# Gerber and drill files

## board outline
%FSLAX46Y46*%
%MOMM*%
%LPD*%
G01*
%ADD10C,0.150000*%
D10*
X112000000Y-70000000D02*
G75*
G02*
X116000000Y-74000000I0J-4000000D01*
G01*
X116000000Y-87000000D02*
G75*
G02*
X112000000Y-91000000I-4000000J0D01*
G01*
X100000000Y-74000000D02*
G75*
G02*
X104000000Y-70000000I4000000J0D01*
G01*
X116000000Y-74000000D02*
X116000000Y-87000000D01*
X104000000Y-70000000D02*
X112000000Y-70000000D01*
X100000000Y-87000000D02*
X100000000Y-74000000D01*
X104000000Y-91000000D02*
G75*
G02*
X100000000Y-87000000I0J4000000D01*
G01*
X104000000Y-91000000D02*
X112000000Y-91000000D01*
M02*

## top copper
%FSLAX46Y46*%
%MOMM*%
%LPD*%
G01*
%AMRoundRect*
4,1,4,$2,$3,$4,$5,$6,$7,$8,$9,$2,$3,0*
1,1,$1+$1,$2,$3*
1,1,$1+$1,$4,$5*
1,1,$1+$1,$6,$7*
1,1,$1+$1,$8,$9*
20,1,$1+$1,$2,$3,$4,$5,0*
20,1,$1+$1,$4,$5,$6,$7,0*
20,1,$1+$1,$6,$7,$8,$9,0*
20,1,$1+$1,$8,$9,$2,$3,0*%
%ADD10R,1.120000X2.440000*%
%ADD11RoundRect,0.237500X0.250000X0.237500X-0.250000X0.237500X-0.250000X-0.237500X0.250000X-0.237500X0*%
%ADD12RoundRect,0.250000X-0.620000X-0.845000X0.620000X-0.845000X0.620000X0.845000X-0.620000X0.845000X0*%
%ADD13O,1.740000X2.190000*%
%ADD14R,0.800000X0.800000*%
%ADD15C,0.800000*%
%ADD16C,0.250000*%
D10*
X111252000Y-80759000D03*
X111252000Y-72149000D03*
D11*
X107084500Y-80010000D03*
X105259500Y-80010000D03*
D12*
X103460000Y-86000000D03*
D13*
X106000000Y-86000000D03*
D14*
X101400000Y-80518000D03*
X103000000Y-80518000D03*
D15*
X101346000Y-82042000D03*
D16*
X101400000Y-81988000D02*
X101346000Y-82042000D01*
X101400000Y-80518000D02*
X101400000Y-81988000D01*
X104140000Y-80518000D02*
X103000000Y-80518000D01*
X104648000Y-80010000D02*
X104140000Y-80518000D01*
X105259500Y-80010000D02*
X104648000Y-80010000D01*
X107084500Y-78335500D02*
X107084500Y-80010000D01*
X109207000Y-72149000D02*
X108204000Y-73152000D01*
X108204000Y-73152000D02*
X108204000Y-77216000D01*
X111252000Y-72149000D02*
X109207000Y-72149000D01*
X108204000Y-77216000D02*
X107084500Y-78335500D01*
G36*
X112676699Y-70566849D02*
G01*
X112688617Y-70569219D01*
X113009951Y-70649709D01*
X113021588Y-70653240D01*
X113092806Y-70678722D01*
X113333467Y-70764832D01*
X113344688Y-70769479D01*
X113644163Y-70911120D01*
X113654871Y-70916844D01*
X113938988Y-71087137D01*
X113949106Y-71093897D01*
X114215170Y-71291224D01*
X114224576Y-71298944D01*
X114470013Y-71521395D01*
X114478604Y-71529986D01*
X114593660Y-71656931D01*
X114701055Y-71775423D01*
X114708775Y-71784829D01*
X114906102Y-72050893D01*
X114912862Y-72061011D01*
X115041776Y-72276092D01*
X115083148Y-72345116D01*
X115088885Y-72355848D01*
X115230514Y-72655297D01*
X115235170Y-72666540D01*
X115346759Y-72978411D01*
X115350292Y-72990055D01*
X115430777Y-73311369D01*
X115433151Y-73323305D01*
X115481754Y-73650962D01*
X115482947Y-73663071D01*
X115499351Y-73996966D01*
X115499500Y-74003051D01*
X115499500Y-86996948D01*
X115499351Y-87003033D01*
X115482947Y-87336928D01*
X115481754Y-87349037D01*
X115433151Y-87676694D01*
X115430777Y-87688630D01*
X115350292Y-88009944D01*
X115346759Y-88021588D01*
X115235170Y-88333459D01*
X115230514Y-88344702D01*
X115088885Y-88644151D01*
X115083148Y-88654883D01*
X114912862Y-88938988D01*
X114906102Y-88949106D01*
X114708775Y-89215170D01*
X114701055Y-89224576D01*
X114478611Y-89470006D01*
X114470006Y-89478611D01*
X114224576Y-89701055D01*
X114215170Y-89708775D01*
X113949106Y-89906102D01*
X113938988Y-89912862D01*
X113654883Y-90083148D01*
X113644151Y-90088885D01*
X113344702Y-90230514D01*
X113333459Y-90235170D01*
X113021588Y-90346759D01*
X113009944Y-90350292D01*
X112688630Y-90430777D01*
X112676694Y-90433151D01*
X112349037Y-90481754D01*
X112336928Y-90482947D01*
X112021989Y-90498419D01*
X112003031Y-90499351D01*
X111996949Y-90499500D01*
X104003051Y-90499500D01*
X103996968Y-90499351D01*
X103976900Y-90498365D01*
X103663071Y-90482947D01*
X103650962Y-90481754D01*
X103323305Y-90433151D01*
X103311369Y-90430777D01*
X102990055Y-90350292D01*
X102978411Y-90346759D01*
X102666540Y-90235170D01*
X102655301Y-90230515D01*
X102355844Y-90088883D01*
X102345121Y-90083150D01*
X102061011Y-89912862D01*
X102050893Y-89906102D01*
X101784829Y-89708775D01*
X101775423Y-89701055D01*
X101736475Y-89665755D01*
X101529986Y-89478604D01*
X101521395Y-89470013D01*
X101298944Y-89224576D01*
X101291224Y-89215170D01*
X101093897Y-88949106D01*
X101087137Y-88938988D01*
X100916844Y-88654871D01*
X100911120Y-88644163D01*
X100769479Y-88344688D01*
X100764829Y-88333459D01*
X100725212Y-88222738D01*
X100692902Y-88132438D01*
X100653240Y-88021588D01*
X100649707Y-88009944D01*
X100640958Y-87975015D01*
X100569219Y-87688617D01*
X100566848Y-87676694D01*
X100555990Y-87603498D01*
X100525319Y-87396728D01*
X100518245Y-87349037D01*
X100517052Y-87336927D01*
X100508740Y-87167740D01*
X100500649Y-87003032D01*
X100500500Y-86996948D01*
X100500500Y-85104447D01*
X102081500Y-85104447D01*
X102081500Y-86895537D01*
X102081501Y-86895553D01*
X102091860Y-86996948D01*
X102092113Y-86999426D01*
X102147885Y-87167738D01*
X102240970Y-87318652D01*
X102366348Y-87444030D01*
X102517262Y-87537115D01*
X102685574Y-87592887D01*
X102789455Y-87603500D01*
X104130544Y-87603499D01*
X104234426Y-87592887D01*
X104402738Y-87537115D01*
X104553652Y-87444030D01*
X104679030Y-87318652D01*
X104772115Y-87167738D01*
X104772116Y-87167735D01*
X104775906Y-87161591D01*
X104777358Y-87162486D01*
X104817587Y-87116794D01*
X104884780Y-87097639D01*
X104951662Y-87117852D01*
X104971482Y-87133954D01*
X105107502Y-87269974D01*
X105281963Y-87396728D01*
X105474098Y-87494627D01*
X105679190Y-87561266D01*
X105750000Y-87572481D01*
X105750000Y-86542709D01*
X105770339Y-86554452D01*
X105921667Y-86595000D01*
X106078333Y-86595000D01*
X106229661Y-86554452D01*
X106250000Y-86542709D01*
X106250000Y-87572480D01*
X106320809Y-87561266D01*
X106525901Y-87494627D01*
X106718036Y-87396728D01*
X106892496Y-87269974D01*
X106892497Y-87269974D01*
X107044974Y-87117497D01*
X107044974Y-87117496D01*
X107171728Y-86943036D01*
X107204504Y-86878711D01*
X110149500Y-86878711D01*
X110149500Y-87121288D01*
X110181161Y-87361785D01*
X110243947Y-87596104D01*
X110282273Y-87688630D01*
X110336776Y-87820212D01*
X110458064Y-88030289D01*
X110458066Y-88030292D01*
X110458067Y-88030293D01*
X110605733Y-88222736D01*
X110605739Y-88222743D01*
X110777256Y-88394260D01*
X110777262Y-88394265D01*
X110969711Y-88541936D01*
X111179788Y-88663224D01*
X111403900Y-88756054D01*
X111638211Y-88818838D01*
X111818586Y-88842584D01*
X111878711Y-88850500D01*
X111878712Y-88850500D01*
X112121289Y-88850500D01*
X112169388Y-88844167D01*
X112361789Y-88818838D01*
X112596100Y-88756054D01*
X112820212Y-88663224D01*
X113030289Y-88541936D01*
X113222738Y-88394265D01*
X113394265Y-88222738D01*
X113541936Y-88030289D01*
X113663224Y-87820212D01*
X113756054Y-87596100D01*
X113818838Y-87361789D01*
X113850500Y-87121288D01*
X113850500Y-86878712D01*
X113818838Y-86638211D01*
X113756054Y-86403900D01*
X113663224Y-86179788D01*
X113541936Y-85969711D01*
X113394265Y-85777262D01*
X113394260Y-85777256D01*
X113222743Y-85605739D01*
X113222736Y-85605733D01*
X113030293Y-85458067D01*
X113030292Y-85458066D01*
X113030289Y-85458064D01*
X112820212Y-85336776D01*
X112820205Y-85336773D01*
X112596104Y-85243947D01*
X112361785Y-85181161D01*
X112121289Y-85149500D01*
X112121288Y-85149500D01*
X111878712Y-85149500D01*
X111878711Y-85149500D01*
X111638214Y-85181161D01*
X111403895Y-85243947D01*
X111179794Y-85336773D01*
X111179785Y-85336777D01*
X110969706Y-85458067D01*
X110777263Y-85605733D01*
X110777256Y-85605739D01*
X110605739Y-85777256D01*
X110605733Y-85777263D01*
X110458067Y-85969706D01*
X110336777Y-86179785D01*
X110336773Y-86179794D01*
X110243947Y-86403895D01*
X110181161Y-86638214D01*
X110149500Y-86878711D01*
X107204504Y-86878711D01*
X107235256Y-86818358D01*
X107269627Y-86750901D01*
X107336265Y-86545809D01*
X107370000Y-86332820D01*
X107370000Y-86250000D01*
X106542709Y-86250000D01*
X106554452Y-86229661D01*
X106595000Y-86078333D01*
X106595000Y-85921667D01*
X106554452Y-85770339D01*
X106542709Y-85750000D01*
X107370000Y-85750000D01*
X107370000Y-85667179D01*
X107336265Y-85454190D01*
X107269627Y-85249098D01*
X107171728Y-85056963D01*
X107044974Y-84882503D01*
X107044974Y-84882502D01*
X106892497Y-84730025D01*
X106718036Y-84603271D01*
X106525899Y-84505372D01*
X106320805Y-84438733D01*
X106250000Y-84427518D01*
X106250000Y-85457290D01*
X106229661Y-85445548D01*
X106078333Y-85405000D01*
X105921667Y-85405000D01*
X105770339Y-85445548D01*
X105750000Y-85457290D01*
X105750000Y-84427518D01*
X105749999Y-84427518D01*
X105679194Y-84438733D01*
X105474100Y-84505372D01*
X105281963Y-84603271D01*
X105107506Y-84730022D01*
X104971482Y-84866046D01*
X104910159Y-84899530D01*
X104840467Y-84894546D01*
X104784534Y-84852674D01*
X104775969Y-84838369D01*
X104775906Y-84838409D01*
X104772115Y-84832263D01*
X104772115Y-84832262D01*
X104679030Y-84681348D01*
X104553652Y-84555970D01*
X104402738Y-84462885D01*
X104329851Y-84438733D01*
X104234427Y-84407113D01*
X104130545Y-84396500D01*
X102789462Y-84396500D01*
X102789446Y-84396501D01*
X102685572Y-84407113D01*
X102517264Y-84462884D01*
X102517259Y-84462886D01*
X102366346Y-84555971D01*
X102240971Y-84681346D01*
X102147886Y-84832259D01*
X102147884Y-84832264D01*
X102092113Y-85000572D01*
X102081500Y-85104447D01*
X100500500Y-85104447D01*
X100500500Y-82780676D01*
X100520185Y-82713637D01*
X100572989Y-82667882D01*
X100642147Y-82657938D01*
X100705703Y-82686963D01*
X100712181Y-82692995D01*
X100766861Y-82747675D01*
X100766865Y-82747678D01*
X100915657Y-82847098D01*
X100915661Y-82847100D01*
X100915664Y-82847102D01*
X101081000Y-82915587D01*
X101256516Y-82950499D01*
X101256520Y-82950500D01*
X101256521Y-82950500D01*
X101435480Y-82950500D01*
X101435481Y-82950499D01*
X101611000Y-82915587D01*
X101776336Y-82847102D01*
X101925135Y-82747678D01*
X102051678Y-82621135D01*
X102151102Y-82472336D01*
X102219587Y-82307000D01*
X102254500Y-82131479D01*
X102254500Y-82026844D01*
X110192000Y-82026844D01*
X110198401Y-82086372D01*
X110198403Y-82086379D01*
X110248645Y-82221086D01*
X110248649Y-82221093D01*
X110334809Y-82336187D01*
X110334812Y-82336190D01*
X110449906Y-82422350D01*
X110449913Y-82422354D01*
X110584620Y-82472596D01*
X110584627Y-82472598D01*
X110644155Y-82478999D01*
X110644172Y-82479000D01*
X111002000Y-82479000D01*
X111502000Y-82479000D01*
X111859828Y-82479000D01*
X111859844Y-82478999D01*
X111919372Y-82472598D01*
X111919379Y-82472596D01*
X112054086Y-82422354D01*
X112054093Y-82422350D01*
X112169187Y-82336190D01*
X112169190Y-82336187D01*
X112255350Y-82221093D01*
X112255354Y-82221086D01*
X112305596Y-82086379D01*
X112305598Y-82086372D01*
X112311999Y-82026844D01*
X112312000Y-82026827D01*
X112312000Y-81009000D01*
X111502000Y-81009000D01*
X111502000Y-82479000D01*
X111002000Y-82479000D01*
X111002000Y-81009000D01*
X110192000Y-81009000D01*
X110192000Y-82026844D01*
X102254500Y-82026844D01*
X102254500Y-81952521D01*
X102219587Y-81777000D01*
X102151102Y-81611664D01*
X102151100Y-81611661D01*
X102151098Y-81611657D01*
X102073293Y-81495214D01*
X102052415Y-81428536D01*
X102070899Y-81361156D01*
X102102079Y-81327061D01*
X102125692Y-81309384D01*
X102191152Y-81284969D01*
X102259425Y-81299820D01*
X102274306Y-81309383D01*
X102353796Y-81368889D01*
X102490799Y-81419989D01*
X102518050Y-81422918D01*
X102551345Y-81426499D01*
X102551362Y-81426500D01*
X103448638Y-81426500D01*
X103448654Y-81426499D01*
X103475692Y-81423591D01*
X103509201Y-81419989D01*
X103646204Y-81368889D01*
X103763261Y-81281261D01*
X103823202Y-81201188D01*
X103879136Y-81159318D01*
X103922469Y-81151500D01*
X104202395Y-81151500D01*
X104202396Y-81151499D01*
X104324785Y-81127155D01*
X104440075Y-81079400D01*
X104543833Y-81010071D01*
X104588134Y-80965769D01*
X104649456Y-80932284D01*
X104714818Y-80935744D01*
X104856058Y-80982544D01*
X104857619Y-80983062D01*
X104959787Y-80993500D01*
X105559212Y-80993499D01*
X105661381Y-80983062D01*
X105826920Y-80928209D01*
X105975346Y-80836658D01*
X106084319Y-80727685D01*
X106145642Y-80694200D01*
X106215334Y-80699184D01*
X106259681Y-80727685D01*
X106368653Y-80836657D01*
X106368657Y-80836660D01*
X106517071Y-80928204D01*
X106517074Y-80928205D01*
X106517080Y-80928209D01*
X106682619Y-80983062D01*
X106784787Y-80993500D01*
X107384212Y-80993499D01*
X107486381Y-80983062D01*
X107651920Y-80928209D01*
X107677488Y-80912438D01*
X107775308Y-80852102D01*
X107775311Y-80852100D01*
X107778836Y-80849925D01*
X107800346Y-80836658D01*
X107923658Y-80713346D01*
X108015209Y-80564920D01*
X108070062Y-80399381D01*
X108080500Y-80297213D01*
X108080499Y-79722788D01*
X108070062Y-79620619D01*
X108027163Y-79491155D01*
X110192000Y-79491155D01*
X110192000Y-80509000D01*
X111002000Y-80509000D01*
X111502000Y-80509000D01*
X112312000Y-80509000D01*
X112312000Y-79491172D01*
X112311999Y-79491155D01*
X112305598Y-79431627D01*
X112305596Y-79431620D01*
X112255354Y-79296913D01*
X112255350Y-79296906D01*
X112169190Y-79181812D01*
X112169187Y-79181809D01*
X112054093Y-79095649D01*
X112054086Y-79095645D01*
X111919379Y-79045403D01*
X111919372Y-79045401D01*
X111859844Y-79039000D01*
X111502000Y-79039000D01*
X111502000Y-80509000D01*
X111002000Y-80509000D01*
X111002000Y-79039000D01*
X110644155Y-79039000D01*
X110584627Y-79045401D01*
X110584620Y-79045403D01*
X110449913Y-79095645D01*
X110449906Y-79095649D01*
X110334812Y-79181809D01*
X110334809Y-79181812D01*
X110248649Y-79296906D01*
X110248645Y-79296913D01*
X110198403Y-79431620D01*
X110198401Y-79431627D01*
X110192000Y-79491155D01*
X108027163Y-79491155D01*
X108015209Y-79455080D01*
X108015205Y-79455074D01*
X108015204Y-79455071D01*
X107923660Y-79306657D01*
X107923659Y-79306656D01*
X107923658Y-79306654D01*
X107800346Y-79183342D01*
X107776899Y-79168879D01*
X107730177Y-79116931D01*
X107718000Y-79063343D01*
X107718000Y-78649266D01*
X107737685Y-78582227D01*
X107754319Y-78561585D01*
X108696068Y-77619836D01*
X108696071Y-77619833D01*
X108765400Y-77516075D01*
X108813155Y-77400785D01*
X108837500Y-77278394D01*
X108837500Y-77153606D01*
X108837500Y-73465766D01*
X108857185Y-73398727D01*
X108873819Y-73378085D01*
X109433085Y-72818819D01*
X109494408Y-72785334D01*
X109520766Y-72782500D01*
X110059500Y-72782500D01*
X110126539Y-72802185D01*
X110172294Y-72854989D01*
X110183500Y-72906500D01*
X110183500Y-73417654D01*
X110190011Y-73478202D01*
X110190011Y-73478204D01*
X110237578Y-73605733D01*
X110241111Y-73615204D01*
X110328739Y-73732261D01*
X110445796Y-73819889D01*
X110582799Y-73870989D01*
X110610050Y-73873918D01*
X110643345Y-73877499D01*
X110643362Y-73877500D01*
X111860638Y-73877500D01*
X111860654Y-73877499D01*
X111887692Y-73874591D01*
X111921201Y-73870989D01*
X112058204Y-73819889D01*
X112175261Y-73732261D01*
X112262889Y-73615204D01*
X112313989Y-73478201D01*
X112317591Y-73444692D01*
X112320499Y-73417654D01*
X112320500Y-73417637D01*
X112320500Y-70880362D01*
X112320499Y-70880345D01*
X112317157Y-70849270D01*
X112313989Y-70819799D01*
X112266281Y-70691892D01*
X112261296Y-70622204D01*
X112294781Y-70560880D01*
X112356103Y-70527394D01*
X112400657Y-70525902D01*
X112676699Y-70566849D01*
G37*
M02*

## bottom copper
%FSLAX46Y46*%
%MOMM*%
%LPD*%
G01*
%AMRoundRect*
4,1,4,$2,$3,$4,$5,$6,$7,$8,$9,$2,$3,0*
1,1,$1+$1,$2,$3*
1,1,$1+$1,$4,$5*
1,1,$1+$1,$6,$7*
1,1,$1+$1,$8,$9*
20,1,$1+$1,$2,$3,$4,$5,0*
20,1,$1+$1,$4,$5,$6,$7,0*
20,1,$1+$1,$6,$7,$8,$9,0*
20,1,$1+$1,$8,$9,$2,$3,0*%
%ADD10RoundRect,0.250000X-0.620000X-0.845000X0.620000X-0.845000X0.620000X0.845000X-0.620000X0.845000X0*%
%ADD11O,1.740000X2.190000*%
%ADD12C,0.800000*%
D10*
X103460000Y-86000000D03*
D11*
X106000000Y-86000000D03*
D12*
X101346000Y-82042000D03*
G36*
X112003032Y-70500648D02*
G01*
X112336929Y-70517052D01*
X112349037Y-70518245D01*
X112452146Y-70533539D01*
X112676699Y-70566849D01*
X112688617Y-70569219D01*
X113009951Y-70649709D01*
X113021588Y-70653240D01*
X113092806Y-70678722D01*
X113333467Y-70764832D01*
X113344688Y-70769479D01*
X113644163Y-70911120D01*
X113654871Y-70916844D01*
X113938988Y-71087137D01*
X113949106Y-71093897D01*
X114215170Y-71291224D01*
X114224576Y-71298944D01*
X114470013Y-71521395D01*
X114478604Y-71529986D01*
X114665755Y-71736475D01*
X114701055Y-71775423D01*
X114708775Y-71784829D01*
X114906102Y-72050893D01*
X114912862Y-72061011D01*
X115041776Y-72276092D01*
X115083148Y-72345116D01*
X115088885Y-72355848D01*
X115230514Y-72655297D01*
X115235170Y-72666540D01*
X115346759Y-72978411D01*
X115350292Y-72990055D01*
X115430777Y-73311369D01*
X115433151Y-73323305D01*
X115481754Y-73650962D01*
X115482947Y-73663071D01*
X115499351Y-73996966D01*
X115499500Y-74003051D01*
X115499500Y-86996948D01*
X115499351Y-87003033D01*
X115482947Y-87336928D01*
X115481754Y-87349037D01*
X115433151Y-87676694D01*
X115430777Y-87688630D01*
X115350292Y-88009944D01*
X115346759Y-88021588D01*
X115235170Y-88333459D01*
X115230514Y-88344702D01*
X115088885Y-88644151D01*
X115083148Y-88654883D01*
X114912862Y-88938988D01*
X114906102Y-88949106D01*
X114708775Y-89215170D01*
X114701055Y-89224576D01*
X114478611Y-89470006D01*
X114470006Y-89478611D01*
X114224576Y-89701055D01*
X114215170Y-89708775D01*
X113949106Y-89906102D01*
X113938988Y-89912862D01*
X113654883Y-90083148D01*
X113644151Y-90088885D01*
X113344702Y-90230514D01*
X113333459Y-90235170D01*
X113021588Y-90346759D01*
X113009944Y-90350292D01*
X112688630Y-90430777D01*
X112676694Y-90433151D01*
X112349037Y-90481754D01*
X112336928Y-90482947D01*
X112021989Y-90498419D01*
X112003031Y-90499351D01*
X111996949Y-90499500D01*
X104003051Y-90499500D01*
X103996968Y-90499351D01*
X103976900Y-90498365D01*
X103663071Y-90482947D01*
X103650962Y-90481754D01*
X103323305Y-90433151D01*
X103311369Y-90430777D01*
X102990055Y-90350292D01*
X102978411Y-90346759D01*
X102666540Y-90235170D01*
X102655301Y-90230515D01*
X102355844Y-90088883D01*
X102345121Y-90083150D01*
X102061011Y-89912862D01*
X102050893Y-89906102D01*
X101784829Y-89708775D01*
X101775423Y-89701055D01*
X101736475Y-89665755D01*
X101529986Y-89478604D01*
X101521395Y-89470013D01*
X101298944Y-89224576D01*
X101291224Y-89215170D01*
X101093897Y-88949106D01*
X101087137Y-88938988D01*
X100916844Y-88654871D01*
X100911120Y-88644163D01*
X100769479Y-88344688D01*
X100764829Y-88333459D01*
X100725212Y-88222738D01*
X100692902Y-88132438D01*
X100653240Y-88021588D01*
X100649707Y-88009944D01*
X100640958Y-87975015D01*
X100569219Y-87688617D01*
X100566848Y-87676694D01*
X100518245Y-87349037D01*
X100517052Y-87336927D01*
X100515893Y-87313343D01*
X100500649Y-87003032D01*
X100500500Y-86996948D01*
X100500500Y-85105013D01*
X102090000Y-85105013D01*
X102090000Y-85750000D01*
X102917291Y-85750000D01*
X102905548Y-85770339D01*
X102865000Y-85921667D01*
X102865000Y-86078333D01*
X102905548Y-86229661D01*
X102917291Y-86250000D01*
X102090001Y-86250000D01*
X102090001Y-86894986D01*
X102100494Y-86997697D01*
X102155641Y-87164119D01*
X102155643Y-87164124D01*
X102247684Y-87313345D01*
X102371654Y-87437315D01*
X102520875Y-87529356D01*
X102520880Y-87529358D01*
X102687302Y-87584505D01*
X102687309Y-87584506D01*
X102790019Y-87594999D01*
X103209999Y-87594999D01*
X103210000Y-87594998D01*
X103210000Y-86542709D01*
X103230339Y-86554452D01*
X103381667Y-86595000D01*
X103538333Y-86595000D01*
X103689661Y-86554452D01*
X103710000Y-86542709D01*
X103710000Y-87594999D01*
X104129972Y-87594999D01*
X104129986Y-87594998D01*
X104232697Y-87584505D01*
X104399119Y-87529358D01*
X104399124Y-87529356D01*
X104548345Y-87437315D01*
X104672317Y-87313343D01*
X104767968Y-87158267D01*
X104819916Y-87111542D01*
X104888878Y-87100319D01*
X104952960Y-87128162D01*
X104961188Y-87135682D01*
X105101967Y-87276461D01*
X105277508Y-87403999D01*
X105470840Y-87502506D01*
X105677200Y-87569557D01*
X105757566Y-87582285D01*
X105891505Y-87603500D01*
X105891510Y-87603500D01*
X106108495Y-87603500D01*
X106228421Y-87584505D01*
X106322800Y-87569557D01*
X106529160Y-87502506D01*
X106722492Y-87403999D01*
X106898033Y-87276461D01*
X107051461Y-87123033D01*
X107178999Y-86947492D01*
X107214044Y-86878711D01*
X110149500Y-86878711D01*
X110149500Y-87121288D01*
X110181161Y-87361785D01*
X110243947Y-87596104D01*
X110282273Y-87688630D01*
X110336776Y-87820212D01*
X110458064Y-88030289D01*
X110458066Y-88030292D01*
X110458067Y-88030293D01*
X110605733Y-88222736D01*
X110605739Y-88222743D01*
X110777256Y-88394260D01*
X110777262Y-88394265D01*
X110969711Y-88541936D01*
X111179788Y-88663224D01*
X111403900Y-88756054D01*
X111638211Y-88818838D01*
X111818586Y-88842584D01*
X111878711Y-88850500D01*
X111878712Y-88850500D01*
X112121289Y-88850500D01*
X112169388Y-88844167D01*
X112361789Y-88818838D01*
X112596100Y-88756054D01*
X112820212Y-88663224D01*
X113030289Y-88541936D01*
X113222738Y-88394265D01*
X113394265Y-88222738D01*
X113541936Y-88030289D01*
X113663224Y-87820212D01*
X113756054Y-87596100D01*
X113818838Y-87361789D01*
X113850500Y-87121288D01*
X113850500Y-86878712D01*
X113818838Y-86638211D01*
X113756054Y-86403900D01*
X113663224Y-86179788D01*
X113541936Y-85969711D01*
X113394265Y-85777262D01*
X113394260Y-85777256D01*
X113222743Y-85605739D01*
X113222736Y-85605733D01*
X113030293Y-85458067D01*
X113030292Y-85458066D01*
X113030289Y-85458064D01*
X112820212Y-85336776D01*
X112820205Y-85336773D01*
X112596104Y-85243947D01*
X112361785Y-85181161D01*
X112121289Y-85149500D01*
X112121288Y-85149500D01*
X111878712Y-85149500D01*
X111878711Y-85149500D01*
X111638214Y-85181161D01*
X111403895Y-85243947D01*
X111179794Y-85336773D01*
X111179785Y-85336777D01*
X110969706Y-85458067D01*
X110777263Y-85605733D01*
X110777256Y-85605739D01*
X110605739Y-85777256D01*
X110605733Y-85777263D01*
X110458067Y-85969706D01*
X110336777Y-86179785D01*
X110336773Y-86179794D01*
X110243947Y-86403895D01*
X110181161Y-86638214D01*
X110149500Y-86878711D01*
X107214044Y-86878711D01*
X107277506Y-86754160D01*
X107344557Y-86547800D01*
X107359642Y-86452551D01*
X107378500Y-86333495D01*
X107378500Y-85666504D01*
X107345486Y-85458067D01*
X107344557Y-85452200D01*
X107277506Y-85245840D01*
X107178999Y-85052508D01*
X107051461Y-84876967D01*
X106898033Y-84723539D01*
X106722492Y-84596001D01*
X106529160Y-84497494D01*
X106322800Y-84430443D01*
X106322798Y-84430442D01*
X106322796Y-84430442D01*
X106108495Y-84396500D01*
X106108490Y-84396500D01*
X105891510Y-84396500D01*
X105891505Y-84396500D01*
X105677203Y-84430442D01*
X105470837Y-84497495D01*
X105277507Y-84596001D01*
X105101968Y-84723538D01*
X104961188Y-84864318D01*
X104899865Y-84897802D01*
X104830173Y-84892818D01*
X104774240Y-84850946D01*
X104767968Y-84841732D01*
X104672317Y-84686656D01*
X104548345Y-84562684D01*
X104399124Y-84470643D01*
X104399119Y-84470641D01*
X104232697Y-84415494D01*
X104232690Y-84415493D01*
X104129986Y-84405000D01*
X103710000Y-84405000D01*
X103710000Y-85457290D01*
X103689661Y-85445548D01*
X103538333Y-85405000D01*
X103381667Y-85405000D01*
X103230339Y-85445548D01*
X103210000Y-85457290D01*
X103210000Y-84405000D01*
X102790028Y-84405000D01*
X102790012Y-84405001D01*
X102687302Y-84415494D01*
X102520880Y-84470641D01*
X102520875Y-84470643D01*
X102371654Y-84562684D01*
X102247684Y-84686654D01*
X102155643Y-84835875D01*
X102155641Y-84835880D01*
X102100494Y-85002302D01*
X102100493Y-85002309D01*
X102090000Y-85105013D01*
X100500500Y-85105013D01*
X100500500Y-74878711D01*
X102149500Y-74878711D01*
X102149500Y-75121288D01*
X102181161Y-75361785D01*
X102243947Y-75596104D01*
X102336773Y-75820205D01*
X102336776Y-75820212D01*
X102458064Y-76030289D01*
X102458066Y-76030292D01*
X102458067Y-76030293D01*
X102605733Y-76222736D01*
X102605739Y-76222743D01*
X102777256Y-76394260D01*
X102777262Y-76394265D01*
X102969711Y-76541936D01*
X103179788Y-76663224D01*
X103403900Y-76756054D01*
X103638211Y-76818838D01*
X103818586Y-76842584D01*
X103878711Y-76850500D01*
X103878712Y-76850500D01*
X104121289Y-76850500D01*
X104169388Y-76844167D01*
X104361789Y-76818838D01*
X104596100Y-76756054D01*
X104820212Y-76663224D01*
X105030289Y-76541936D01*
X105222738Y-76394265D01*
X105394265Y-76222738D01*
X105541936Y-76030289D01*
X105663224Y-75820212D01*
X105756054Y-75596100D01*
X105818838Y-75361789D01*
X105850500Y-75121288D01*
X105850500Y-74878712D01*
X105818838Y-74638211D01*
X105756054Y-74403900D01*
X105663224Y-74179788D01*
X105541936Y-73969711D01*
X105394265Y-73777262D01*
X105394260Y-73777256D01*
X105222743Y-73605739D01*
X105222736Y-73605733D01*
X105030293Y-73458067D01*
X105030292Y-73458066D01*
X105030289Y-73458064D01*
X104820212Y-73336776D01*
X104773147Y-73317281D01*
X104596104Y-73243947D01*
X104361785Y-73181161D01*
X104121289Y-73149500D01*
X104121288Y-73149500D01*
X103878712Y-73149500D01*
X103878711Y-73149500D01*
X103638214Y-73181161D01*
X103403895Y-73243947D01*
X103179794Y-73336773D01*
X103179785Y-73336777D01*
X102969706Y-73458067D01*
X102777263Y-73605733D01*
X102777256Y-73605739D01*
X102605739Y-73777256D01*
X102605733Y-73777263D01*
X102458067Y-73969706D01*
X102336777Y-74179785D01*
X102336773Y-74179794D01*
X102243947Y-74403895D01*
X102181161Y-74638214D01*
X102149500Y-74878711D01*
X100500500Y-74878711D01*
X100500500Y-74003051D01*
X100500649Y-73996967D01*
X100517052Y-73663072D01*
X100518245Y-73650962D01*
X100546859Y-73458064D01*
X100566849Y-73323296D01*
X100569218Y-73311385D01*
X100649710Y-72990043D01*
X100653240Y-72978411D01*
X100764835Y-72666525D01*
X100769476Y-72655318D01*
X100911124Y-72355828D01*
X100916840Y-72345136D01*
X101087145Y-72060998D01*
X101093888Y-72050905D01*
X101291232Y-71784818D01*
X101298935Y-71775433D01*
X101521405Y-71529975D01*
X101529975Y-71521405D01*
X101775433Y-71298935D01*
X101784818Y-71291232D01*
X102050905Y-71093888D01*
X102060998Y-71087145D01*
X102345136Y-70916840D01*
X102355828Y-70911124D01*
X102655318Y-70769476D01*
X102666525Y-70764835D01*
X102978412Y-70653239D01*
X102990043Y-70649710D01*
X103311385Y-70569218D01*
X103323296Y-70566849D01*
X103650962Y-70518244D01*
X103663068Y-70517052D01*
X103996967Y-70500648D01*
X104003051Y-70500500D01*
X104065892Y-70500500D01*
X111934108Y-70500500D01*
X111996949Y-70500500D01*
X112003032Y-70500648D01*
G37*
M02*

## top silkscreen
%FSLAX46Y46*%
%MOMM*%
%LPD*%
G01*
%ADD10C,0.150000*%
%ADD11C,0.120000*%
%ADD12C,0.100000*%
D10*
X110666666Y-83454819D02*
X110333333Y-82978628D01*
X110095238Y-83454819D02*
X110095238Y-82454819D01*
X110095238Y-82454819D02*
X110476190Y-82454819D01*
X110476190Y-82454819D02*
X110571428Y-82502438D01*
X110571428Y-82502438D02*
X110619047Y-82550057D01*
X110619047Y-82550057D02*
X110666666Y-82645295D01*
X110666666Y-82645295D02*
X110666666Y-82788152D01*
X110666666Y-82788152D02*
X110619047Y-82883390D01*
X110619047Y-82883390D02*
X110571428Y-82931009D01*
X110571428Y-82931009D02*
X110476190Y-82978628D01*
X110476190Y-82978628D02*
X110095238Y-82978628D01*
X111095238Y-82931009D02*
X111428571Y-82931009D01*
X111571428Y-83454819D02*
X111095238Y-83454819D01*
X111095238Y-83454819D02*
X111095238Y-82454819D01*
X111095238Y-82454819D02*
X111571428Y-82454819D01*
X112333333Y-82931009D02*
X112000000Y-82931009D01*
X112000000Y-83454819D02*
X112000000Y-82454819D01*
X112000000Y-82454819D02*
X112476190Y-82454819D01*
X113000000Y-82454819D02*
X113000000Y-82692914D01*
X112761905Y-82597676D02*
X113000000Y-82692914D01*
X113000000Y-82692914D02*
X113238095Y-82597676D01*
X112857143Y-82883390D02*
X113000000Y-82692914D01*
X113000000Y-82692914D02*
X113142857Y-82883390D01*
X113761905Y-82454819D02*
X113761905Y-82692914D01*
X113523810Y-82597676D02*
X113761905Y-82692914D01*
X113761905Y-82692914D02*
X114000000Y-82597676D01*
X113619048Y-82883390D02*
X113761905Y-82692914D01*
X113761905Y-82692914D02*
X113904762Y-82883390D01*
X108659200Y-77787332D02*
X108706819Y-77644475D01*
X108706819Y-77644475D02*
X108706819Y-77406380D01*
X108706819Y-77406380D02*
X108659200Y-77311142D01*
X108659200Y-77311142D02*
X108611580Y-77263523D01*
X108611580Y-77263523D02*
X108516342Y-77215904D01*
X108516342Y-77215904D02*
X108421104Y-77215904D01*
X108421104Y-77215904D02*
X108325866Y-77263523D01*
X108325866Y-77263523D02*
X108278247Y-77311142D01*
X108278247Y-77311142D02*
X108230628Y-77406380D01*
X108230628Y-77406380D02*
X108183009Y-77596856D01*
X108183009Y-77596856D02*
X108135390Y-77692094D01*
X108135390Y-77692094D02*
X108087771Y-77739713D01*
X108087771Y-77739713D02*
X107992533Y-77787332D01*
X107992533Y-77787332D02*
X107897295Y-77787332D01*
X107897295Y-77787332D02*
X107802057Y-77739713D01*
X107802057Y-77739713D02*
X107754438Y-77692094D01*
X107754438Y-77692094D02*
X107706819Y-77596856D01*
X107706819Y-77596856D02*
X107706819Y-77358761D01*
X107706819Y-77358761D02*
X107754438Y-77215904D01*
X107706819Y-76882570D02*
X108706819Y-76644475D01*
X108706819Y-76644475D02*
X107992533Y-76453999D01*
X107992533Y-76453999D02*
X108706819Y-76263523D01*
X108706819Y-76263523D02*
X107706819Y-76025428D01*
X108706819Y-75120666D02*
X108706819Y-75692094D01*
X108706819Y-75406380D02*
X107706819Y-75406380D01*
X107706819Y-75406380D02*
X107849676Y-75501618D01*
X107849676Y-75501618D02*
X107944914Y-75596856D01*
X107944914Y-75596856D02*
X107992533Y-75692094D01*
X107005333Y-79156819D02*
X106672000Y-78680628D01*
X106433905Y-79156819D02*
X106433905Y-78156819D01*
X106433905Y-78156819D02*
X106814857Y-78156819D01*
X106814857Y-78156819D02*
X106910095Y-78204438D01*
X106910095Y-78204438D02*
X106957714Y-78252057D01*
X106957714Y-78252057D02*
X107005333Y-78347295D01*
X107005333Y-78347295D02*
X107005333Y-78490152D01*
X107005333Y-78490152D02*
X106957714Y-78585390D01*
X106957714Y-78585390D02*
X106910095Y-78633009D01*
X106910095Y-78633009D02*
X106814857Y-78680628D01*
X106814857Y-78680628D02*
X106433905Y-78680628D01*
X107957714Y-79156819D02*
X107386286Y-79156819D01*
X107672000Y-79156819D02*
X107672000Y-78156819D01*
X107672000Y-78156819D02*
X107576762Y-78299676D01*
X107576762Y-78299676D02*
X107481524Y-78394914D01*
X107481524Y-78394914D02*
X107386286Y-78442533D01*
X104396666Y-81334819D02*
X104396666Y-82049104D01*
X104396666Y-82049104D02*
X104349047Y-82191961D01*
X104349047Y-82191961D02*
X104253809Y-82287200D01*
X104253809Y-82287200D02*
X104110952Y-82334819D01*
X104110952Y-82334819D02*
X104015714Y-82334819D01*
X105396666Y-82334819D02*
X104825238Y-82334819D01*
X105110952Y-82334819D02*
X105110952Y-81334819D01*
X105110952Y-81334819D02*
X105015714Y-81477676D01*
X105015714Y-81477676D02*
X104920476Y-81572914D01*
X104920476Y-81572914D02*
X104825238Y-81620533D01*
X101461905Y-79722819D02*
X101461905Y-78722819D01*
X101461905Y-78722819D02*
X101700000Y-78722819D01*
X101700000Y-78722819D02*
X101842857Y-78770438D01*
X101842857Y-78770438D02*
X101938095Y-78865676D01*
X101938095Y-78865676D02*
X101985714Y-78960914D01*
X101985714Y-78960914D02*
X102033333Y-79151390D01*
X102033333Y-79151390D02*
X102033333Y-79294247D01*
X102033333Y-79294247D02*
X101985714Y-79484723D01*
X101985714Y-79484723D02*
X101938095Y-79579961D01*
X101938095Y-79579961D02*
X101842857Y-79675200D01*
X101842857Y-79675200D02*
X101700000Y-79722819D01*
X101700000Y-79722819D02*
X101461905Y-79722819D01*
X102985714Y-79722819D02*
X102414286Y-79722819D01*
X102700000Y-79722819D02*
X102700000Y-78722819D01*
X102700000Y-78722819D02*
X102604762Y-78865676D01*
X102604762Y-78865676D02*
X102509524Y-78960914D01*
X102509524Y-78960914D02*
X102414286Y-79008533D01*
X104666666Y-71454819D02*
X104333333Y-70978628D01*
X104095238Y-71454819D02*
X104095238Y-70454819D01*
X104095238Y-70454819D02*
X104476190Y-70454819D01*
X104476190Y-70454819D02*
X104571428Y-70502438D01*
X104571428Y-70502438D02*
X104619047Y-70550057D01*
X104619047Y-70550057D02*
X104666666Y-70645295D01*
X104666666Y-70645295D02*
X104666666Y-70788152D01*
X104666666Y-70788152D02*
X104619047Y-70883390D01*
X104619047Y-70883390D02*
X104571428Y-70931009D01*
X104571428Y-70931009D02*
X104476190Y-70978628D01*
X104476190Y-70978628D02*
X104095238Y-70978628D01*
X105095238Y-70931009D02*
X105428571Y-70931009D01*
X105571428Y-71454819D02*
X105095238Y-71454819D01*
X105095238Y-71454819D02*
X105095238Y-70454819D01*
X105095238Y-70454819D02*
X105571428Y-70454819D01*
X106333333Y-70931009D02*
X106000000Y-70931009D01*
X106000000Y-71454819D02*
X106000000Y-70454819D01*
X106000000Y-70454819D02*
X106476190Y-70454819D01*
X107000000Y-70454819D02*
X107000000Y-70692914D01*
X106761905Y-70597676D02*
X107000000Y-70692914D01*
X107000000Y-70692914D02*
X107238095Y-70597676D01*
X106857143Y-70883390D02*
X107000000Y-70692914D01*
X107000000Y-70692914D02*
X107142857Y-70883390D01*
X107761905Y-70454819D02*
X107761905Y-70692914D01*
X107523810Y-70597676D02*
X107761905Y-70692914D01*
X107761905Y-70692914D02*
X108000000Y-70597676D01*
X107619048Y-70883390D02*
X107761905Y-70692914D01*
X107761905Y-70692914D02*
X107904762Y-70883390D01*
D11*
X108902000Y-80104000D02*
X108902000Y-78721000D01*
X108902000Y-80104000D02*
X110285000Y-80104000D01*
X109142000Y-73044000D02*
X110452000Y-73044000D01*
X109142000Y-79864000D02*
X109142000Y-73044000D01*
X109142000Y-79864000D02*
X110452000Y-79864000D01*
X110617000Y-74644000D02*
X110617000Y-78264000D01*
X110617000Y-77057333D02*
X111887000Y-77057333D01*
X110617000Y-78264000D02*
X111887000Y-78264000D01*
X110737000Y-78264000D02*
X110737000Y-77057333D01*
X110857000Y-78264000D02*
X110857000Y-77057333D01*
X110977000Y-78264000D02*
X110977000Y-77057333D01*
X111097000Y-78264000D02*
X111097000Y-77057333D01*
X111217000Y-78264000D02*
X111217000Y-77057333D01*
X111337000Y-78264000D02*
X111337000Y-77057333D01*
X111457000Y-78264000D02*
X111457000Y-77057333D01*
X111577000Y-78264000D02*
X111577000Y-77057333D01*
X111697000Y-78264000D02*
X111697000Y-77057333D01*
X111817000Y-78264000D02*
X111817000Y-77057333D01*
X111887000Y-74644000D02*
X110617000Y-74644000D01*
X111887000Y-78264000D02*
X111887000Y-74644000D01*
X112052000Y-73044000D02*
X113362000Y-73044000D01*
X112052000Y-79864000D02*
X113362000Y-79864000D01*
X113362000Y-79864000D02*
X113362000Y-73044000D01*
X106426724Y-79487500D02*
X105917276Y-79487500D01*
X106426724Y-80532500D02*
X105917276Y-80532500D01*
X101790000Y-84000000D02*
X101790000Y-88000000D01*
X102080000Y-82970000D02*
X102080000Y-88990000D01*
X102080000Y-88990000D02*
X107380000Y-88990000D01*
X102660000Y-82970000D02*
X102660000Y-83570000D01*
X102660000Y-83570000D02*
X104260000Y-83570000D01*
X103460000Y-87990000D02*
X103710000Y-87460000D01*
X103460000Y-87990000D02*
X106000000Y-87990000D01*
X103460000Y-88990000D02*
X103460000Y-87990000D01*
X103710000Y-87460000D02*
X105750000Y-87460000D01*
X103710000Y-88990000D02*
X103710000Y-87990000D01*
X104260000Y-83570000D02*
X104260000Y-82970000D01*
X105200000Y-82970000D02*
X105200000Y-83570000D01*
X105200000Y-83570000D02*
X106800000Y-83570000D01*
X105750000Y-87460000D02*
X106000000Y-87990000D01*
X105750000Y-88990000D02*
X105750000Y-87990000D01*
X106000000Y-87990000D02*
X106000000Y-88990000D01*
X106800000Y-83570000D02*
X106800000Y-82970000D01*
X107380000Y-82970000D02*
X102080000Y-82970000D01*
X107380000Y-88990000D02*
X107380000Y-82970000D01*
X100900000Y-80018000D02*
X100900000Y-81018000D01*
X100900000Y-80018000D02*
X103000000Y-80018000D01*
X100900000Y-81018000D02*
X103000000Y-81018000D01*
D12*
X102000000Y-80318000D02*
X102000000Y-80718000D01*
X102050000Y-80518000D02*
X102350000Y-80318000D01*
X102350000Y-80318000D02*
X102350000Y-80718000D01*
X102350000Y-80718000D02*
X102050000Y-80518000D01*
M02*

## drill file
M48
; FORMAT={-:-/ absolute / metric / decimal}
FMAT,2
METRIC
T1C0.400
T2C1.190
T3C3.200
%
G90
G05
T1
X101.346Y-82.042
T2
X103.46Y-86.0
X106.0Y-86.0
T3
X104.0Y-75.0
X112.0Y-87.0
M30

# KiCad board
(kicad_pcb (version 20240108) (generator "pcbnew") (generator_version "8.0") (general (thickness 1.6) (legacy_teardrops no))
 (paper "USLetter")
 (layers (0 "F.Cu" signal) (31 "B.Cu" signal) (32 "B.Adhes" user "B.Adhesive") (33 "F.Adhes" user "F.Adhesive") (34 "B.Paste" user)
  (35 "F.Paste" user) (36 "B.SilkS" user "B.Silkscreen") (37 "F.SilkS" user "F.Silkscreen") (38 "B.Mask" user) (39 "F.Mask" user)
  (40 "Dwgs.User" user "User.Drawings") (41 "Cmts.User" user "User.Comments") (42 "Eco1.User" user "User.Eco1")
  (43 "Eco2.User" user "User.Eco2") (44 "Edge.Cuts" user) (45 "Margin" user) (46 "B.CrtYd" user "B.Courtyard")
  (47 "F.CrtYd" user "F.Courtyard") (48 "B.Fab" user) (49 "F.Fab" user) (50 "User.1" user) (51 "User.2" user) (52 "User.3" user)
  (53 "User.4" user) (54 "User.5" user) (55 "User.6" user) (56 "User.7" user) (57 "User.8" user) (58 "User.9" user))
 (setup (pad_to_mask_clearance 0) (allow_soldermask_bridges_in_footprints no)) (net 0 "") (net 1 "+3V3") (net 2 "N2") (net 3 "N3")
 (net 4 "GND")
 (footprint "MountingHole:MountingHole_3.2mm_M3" (layer "F.Cu") (at 112 87)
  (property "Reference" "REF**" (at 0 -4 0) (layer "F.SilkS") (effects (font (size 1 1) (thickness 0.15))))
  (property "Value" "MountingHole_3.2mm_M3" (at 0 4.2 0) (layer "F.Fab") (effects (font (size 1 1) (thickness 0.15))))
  (pad "" np_thru_hole circle (at 0 0) (size 3.2 3.2) (drill 3.2) (layers "*.Cu" "*.Mask")))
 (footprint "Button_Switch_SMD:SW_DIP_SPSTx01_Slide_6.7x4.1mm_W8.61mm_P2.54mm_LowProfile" (layer "F.Cu") (at 111.252 76.454 90)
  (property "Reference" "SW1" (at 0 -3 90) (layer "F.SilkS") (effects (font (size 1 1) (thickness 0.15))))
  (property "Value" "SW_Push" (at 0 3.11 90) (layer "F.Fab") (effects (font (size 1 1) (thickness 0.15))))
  (fp_line (start -3.65 -2.35) (end -2.267 -2.35) (stroke (width 0.12) (type solid)) (layer "F.SilkS"))
  (fp_line (start -3.65 -2.35) (end -3.65 -0.967) (stroke (width 0.12) (type solid)) (layer "F.SilkS"))
  (fp_line (start 3.41 -2.11) (end 3.41 -0.8) (stroke (width 0.12) (type solid)) (layer "F.SilkS"))
  (fp_line (start -3.41 -2.11) (end 3.41 -2.11) (stroke (width 0.12) (type solid)) (layer "F.SilkS"))
  (fp_line (start -3.41 -2.11) (end -3.41 -0.8) (stroke (width 0.12) (type solid)) (layer "F.SilkS"))
  (fp_line (start 1.81 -0.635) (end -1.81 -0.635) (stroke (width 0.12) (type solid)) (layer "F.SilkS"))
  (fp_line (start -0.603333 -0.635) (end -0.603333 0.635) (stroke (width 0.12) (type solid)) (layer "F.SilkS"))
  (fp_line (start -1.81 -0.635) (end -1.81 0.635) (stroke (width 0.12) (type solid)) (layer "F.SilkS"))
  (fp_line (start -1.81 -0.515) (end -0.603333 -0.515) (stroke (width 0.12) (type solid)) (layer "F.SilkS"))
  (fp_line (start -1.81 -0.395) (end -0.603333 -0.395) (stroke (width 0.12) (type solid)) (layer "F.SilkS"))
  (fp_line (start -1.81 -0.275) (end -0.603333 -0.275) (stroke (width 0.12) (type solid)) (layer "F.SilkS"))
  (fp_line (start -1.81 -0.155) (end -0.603333 -0.155) (stroke (width 0.12) (type solid)) (layer "F.SilkS"))
  (fp_line (start -1.81 -0.035) (end -0.603333 -0.035) (stroke (width 0.12) (type solid)) (layer "F.SilkS"))
  (fp_line (start -1.81 0.085) (end -0.603333 0.085) (stroke (width 0.12) (type solid)) (layer "F.SilkS"))
  (fp_line (start -1.81 0.205) (end -0.603333 0.205) (stroke (width 0.12) (type solid)) (layer "F.SilkS"))
  (fp_line (start -1.81 0.325) (end -0.603333 0.325) (stroke (width 0.12) (type solid)) (layer "F.SilkS"))
  (fp_line (start -1.81 0.445) (end -0.603333 0.445) (stroke (width 0.12) (type solid)) (layer "F.SilkS"))
  (fp_line (start -1.81 0.565) (end -0.603333 0.565) (stroke (width 0.12) (type solid)) (layer "F.SilkS"))
  (fp_line (start 1.81 0.635) (end 1.81 -0.635) (stroke (width 0.12) (type solid)) (layer "F.SilkS"))
  (fp_line (start -1.81 0.635) (end 1.81 0.635) (stroke (width 0.12) (type solid)) (layer "F.SilkS"))
  (fp_line (start 3.41 0.8) (end 3.41 2.11) (stroke (width 0.12) (type solid)) (layer "F.SilkS"))
  (fp_line (start -3.41 0.8) (end -3.41 2.11) (stroke (width 0.12) (type solid)) (layer "F.SilkS"))
  (fp_line (start -3.41 2.11) (end 3.41 2.11) (stroke (width 0.12) (type solid)) (layer "F.SilkS"))
  (pad "1" smd rect (at -4.305 0 90) (size 2.44 1.12) (layers "F.Cu" "F.Paste" "F.Mask") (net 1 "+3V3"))
  (pad "2" smd rect (at 4.305 0 90) (size 2.44 1.12) (layers "F.Cu" "F.Paste" "F.Mask") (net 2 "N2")))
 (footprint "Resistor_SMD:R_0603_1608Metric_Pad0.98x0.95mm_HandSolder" (layer "F.Cu") (at 106.172 80.01 180)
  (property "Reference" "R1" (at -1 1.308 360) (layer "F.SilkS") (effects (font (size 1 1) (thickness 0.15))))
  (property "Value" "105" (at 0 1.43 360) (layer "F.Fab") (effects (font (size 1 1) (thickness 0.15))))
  (fp_line (start -0.254724 0.5225) (end 0.254724 0.5225) (stroke (width 0.12) (type solid)) (layer "F.SilkS"))
  (fp_line (start -0.254724 -0.5225) (end 0.254724 -0.5225) (stroke (width 0.12) (type solid)) (layer "F.SilkS"))
  (pad "1" smd roundrect (at -0.9125 0 180) (size 0.975 0.95) (layers "F.Cu" "F.Paste" "F.Mask") (roundrect_rratio 0.25) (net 2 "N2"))
  (pad "2" smd roundrect (at 0.9125 0 180) (size 0.975 0.95) (layers "F.Cu" "F.Paste" "F.Mask") (roundrect_rratio 0.25) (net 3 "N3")))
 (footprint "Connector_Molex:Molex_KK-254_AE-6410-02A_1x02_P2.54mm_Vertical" (layer "F.Cu") (at 103.46 86)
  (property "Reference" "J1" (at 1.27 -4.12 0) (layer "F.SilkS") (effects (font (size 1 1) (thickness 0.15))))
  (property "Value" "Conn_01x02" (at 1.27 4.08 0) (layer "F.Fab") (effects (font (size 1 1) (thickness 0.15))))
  (fp_line (start -1.67 -2) (end -1.67 2) (stroke (width 0.12) (type solid)) (layer "F.SilkS"))
  (fp_line (start -1.38 -3.03) (end -1.38 2.99) (stroke (width 0.12) (type solid)) (layer "F.SilkS"))
  (fp_line (start -1.38 2.99) (end 3.92 2.99) (stroke (width 0.12) (type solid)) (layer "F.SilkS"))
  (fp_line (start -0.8 -3.03) (end -0.8 -2.43) (stroke (width 0.12) (type solid)) (layer "F.SilkS"))
  (fp_line (start -0.8 -2.43) (end 0.8 -2.43) (stroke (width 0.12) (type solid)) (layer "F.SilkS"))
  (fp_line (start 0 1.99) (end 0.25 1.46) (stroke (width 0.12) (type solid)) (layer "F.SilkS"))
  (fp_line (start 0 1.99) (end 2.54 1.99) (stroke (width 0.12) (type solid)) (layer "F.SilkS"))
  (fp_line (start 0 2.99) (end 0 1.99) (stroke (width 0.12) (type solid)) (layer "F.SilkS"))
  (fp_line (start 0.25 1.46) (end 2.29 1.46) (stroke (width 0.12) (type solid)) (layer "F.SilkS"))
  (fp_line (start 0.25 2.99) (end 0.25 1.99) (stroke (width 0.12) (type solid)) (layer "F.SilkS"))
  (fp_line (start 0.8 -2.43) (end 0.8 -3.03) (stroke (width 0.12) (type solid)) (layer "F.SilkS"))
  (fp_line (start 1.74 -3.03) (end 1.74 -2.43) (stroke (width 0.12) (type solid)) (layer "F.SilkS"))
  (fp_line (start 1.74 -2.43) (end 3.34 -2.43) (stroke (width 0.12) (type solid)) (layer "F.SilkS"))
  (fp_line (start 2.29 1.46) (end 2.54 1.99) (stroke (width 0.12) (type solid)) (layer "F.SilkS"))
  (fp_line (start 2.29 2.99) (end 2.29 1.99) (stroke (width 0.12) (type solid)) (layer "F.SilkS"))
  (fp_line (start 2.54 1.99) (end 2.54 2.99) (stroke (width 0.12) (type solid)) (layer "F.SilkS"))
  (fp_line (start 3.34 -2.43) (end 3.34 -3.03) (stroke (width 0.12) (type solid)) (layer "F.SilkS"))
  (fp_line (start 3.92 -3.03) (end -1.38 -3.03) (stroke (width 0.12) (type solid)) (layer "F.SilkS"))
  (fp_line (start 3.92 2.99) (end 3.92 -3.03) (stroke (width 0.12) (type solid)) (layer "F.SilkS"))
  (pad "1" thru_hole roundrect (at 0 0) (size 1.74 2.19) (drill 1.19) (layers "*.Cu" "*.Mask") (remove_unused_layers no)
   (roundrect_rratio 0.143678) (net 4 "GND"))
  (pad "2" thru_hole oval (at 2.54 0) (size 1.74 2.19) (drill 1.19) (layers "*.Cu" "*.Mask") (remove_unused_layers no) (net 1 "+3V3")))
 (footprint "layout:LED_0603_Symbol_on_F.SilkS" (layer "F.Cu") (at 102.2 80.518)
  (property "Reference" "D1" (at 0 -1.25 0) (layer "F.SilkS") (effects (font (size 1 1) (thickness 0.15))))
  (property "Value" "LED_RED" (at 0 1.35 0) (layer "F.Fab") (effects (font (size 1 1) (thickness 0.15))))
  (fp_line (start -1.3 -0.5) (end -1.3 0.5) (stroke (width 0.12) (type solid)) (layer "F.SilkS"))
  (fp_line (start -1.3 -0.5) (end 0.8 -0.5) (stroke (width 0.12) (type solid)) (layer "F.SilkS"))
  (fp_line (start -1.3 0.5) (end 0.8 0.5) (stroke (width 0.12) (type solid)) (layer "F.SilkS"))
  (fp_line (start -0.2 -0.2) (end -0.2 0.2) (stroke (width 0.1) (type solid)) (layer "F.SilkS"))
  (fp_line (start -0.15 0) (end 0.15 -0.2) (stroke (width 0.1) (type solid)) (layer "F.SilkS"))
  (fp_line (start 0.15 -0.2) (end 0.15 0.2) (stroke (width 0.1) (type solid)) (layer "F.SilkS"))
  (fp_line (start 0.15 0.2) (end -0.15 0) (stroke (width 0.1) (type solid)) (layer "F.SilkS"))
  (pad "1" smd rect (at -0.8 0 180) (size 0.8 0.8) (layers "F.Cu" "F.Paste" "F.Mask") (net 4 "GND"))
  (pad "2" smd rect (at 0.8 0 180) (size 0.8 0.8) (layers "F.Cu" "F.Paste" "F.Mask") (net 3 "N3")))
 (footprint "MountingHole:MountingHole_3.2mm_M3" (layer "F.Cu") (at 104 75)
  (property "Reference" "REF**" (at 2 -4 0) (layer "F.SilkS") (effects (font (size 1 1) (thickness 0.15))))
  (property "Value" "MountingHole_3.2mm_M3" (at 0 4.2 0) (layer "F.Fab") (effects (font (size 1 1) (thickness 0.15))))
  (pad "" np_thru_hole circle (at 0 0) (size 3.2 3.2) (drill 3.2) (layers "*.Cu" "*.Mask")))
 (gr_arc (start 112 70) (mid 114.828427 71.171573) (end 116 74) (stroke (width 0.15) (type default)) (layer "Edge.Cuts"))
 (gr_arc (start 116 87) (mid 114.828427 89.828427) (end 112 91) (stroke (width 0.15) (type default)) (layer "Edge.Cuts"))
 (gr_arc (start 100 74) (mid 101.171573 71.171573) (end 104 70) (stroke (width 0.15) (type default)) (layer "Edge.Cuts"))
 (gr_line (start 116 74) (end 116 87) (stroke (width 0.15) (type default)) (layer "Edge.Cuts"))
 (gr_line (start 104 70) (end 112 70) (stroke (width 0.15) (type default)) (layer "Edge.Cuts"))
 (gr_line (start 100 87) (end 100 74) (stroke (width 0.15) (type default)) (layer "Edge.Cuts"))
 (gr_arc (start 104 91) (mid 101.171573 89.828427) (end 100 87) (stroke (width 0.15) (type default)) (layer "Edge.Cuts"))
 (gr_line (start 104 91) (end 112 91) (stroke (width 0.15) (type default)) (layer "Edge.Cuts"))
 (segment (start 101.4 81.988) (end 101.346 82.042) (width 0.25) (layer "F.Cu") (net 4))
 (segment (start 101.4 80.518) (end 101.4 81.988) (width 0.25) (layer "F.Cu") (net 4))
 (via (at 101.346 82.042) (size 0.8) (drill 0.4) (layers "F.Cu" "B.Cu") (free yes) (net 4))
 (segment (start 104.14 80.518) (end 103 80.518) (width 0.25) (layer "F.Cu") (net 3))
 (segment (start 104.648 80.01) (end 104.14 80.518) (width 0.25) (layer "F.Cu") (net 3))
 (segment (start 105.2595 80.01) (end 104.648 80.01) (width 0.25) (layer "F.Cu") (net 3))
 (segment (start 107.0845 78.3355) (end 107.0845 80.01) (width 0.25) (layer "F.Cu") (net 2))
 (segment (start 109.207 72.149) (end 108.204 73.152) (width 0.25) (layer "F.Cu") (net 2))
 (segment (start 108.204 73.152) (end 108.204 77.216) (width 0.25) (layer "F.Cu") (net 2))
 (segment (start 111.252 72.149) (end 109.207 72.149) (width 0.25) (layer "F.Cu") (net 2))
 (segment (start 108.204 77.216) (end 107.0845 78.3355) (width 0.25) (layer "F.Cu") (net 2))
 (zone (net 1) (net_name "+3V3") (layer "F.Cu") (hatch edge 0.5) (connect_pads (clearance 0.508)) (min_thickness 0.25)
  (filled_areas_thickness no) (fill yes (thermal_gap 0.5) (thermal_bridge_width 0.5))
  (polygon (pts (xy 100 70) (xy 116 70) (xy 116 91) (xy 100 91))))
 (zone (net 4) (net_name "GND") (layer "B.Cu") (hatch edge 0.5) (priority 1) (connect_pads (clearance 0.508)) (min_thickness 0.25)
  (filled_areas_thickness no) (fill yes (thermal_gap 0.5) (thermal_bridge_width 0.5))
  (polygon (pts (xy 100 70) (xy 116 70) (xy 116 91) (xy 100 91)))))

